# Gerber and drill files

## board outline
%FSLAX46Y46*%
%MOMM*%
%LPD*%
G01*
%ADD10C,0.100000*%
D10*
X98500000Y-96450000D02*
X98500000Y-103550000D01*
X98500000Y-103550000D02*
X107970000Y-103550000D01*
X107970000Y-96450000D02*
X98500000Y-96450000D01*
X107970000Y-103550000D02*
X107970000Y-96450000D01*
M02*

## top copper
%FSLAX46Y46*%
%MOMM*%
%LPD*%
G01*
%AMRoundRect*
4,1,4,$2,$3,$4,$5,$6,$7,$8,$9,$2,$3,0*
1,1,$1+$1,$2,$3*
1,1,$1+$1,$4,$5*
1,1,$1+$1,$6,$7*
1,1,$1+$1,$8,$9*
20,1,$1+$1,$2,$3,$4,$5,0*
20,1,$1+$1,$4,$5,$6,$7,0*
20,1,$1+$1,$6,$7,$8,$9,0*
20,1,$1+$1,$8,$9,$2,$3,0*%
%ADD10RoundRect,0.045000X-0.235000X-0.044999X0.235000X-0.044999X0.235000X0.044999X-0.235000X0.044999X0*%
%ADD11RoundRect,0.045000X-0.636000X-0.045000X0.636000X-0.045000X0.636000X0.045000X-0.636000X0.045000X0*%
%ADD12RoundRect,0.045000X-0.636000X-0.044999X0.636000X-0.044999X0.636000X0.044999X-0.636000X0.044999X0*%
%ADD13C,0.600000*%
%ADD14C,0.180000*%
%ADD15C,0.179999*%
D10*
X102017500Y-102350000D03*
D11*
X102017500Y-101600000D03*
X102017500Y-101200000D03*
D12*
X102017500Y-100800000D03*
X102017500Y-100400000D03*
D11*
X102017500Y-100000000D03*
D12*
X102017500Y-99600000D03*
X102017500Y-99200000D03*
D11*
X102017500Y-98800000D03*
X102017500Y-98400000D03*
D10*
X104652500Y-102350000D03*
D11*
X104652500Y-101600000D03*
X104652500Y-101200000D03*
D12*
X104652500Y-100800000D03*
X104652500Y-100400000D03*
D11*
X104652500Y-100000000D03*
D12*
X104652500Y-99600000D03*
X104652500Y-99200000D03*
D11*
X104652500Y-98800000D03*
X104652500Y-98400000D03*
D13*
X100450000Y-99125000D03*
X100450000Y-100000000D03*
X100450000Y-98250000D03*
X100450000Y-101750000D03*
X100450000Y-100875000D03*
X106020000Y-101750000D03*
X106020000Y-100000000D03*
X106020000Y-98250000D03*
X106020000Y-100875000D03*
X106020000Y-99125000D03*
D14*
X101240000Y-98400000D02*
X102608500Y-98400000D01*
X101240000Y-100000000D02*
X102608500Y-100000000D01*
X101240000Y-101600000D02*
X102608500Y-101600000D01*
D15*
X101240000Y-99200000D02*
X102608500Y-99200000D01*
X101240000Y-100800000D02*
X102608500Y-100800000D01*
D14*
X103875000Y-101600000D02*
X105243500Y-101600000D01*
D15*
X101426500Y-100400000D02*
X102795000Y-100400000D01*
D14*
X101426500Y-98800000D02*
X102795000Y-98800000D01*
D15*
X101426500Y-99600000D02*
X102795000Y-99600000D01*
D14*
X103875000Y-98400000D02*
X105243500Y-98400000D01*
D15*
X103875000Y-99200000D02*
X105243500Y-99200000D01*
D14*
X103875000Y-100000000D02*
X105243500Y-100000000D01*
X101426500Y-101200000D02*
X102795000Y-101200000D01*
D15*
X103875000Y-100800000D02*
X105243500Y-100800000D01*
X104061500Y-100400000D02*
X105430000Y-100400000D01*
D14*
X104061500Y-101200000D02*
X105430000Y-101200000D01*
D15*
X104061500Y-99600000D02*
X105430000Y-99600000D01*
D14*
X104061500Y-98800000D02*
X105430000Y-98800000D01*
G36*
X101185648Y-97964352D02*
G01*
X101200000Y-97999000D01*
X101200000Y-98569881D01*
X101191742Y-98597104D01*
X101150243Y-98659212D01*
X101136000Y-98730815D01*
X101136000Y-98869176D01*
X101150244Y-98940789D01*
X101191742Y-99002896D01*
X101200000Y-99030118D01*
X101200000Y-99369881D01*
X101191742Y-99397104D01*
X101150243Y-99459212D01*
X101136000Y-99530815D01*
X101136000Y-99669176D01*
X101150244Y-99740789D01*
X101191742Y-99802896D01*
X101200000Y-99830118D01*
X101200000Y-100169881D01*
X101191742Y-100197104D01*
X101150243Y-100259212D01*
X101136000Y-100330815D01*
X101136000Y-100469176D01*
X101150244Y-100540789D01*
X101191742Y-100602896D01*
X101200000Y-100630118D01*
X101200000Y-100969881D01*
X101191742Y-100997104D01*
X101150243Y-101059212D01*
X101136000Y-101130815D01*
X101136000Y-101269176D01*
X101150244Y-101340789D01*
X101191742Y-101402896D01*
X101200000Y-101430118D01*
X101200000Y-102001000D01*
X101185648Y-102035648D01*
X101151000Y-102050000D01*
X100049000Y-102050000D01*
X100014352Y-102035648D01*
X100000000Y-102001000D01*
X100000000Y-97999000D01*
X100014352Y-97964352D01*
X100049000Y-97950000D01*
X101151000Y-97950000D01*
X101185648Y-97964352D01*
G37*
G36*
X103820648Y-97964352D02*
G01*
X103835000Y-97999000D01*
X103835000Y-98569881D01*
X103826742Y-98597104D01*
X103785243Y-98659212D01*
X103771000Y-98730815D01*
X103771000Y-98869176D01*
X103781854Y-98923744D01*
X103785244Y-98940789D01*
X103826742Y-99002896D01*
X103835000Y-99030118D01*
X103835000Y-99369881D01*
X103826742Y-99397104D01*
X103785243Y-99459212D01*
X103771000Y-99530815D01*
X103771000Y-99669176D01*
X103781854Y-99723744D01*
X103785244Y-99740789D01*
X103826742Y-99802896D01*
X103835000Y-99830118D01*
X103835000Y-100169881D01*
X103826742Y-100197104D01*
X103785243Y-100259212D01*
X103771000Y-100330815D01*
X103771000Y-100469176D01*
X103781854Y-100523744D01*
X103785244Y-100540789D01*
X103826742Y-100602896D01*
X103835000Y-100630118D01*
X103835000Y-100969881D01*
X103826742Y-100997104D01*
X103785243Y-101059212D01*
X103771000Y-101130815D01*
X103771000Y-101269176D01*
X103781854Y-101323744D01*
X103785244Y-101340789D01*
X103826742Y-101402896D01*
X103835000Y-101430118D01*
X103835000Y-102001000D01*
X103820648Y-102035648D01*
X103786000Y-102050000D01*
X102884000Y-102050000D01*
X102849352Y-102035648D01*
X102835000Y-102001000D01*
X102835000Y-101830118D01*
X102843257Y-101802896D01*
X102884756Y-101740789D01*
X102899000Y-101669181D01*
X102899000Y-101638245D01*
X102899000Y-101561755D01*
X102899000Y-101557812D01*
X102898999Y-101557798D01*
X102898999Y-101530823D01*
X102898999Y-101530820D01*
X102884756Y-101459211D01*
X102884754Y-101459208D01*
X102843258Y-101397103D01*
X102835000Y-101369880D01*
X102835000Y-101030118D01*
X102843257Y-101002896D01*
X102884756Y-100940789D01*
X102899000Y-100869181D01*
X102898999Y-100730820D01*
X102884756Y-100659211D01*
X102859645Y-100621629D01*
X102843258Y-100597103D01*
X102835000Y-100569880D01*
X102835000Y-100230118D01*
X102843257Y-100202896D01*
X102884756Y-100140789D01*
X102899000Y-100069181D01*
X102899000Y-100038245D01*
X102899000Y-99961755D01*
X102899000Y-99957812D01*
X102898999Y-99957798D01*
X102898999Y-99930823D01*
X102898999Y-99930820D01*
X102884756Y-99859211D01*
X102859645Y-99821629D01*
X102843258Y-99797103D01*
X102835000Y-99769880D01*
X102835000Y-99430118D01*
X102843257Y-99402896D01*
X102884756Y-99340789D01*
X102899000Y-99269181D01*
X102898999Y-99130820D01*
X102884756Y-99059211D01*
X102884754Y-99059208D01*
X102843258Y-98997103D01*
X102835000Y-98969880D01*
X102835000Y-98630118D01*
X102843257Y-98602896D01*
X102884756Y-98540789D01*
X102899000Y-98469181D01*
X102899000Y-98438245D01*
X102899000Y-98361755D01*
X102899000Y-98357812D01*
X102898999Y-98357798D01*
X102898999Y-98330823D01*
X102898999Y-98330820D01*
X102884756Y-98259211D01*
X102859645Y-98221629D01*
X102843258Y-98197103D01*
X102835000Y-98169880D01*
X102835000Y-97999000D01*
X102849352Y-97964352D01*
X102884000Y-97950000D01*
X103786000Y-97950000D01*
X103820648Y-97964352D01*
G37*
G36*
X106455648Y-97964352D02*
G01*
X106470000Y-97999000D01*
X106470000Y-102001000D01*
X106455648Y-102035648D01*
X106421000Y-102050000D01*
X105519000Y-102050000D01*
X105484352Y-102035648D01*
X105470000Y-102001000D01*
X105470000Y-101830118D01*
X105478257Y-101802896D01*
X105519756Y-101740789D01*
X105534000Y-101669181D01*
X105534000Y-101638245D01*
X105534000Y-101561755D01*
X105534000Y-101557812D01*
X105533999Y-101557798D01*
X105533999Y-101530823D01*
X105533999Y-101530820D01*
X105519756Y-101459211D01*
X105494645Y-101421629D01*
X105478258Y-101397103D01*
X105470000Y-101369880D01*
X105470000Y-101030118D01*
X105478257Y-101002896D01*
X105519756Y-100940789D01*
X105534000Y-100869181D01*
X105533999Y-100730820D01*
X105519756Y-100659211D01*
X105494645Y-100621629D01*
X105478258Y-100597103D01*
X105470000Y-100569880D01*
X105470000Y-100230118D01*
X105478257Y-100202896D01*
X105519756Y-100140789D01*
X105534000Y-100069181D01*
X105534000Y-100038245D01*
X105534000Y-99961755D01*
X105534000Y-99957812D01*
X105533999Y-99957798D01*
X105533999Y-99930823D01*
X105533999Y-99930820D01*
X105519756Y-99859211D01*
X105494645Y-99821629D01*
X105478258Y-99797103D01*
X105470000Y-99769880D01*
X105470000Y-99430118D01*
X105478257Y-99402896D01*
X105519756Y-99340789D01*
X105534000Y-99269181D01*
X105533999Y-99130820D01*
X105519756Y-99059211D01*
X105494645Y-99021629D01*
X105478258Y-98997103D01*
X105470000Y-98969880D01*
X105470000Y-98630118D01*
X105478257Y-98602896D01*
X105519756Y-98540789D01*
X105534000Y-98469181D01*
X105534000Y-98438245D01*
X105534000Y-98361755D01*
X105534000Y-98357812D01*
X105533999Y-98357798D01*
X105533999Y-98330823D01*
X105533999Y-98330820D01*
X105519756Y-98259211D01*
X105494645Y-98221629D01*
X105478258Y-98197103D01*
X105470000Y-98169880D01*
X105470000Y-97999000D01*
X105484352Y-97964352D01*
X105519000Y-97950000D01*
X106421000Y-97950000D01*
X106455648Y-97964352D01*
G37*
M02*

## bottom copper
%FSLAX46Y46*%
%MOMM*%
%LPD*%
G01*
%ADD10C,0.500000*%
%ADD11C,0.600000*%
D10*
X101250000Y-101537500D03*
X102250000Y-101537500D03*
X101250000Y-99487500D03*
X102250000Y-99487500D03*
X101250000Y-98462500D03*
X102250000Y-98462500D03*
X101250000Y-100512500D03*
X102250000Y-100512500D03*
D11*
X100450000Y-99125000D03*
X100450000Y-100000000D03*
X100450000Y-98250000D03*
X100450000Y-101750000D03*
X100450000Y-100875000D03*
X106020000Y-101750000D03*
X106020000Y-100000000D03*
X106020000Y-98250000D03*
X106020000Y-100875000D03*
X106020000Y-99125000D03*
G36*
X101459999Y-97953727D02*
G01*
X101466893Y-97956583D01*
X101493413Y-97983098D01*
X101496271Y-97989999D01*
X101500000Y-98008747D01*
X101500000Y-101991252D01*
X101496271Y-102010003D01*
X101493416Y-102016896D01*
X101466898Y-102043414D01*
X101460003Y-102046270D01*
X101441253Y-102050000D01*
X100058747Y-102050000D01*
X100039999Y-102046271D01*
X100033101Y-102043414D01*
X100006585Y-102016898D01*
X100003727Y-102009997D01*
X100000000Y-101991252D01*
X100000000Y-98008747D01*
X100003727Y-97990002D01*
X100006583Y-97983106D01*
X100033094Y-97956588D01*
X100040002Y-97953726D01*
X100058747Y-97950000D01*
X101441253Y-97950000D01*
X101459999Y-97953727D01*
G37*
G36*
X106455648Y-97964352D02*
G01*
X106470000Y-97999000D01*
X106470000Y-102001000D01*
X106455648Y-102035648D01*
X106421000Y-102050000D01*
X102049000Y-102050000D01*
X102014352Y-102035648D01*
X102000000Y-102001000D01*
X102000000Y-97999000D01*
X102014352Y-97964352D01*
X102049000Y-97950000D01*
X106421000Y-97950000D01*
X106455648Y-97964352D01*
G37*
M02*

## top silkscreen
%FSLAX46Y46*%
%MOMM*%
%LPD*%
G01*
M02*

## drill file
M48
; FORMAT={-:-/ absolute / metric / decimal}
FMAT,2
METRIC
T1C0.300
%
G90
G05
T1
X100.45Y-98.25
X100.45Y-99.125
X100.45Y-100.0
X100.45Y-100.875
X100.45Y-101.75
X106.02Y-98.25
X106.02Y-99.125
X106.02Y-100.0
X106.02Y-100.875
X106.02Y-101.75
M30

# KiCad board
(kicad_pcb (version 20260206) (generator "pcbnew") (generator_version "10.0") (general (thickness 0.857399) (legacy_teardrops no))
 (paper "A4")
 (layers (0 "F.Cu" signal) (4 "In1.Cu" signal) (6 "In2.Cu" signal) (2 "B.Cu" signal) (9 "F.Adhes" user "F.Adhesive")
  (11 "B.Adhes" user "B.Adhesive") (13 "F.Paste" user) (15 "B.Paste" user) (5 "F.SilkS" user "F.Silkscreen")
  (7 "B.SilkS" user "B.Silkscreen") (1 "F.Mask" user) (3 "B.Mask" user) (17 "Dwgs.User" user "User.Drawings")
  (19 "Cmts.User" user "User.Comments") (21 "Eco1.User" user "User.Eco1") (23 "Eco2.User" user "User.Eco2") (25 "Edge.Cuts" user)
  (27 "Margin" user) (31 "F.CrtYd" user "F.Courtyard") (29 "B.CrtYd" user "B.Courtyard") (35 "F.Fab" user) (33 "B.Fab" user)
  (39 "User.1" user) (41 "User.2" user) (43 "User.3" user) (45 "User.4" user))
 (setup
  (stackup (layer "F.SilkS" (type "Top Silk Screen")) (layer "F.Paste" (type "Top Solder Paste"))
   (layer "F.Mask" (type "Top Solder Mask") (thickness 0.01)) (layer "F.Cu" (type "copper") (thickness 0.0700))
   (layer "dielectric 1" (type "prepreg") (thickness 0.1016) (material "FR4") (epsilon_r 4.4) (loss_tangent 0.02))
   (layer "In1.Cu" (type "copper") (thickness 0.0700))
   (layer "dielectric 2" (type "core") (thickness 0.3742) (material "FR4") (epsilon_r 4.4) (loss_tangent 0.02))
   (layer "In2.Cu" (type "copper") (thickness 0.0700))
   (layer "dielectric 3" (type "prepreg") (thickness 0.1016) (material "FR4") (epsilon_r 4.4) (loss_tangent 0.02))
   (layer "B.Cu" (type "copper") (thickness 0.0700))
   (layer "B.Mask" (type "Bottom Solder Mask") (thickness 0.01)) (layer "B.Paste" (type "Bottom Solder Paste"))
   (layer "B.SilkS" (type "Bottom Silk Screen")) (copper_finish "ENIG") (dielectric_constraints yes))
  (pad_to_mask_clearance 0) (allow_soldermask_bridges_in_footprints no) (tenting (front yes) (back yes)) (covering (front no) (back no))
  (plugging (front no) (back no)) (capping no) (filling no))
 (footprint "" (layer "F.Cu") (at 0 0)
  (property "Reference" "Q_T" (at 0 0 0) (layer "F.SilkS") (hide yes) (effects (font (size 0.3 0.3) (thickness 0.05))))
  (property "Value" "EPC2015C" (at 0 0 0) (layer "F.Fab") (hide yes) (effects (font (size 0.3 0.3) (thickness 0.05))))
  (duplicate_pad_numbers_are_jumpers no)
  (pad "1" smd roundrect (at 102.0175 102.35) (size 0.56 0.179999) (layers "F.Cu" "F.Mask" "F.Paste") (roundrect_rratio 0.25) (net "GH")
   (thermal_bridge_angle 45))
  (pad "3" smd roundrect (at 102.0175 101.6) (size 1.362 0.18) (layers "F.Cu" "F.Mask" "F.Paste") (roundrect_rratio 0.25) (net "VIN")
   (thermal_bridge_angle 45))
  (pad "4" smd roundrect (at 102.0175 101.2) (size 1.362 0.18) (layers "F.Cu" "F.Mask" "F.Paste") (roundrect_rratio 0.25) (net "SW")
   (thermal_bridge_angle 45))
  (pad "5" smd roundrect (at 102.0175 100.8) (size 1.362 0.179999) (layers "F.Cu" "F.Mask" "F.Paste") (roundrect_rratio 0.25) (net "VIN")
   (thermal_bridge_angle 45))
  (pad "6" smd roundrect (at 102.0175 100.4) (size 1.362 0.179999) (layers "F.Cu" "F.Mask" "F.Paste") (roundrect_rratio 0.25) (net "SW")
   (thermal_bridge_angle 45))
  (pad "7" smd roundrect (at 102.0175 100) (size 1.362 0.18) (layers "F.Cu" "F.Mask" "F.Paste") (roundrect_rratio 0.25) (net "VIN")
   (thermal_bridge_angle 45))
  (pad "8" smd roundrect (at 102.0175 99.6) (size 1.362 0.179999) (layers "F.Cu" "F.Mask" "F.Paste") (roundrect_rratio 0.25) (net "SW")
   (thermal_bridge_angle 45))
  (pad "9" smd roundrect (at 102.0175 99.2) (size 1.362 0.179999) (layers "F.Cu" "F.Mask" "F.Paste") (roundrect_rratio 0.25) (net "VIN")
   (thermal_bridge_angle 45))
  (pad "10" smd roundrect (at 102.0175 98.8) (size 1.362 0.18) (layers "F.Cu" "F.Mask" "F.Paste") (roundrect_rratio 0.25) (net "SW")
   (thermal_bridge_angle 45))
  (pad "11" smd roundrect (at 102.0175 98.4) (size 1.362 0.18) (layers "F.Cu" "F.Mask" "F.Paste") (roundrect_rratio 0.25) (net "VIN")
   (thermal_bridge_angle 45)))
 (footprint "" (layer "F.Cu") (at 0 0)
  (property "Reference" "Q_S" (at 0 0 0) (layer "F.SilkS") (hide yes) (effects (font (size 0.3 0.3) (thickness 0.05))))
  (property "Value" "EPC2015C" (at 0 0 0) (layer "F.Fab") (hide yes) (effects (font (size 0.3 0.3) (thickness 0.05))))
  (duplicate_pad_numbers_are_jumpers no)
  (pad "1" smd roundrect (at 104.6525 102.35) (size 0.56 0.179999) (layers "F.Cu" "F.Mask" "F.Paste") (roundrect_rratio 0.25) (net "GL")
   (thermal_bridge_angle 45))
  (pad "3" smd roundrect (at 104.6525 101.6) (size 1.362 0.18) (layers "F.Cu" "F.Mask" "F.Paste") (roundrect_rratio 0.25) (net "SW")
   (thermal_bridge_angle 45))
  (pad "4" smd roundrect (at 104.6525 101.2) (size 1.362 0.18) (layers "F.Cu" "F.Mask" "F.Paste") (roundrect_rratio 0.25) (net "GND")
   (thermal_bridge_angle 45))
  (pad "5" smd roundrect (at 104.6525 100.8) (size 1.362 0.179999) (layers "F.Cu" "F.Mask" "F.Paste") (roundrect_rratio 0.25) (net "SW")
   (thermal_bridge_angle 45))
  (pad "6" smd roundrect (at 104.6525 100.4) (size 1.362 0.179999) (layers "F.Cu" "F.Mask" "F.Paste") (roundrect_rratio 0.25) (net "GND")
   (thermal_bridge_angle 45))
  (pad "7" smd roundrect (at 104.6525 100) (size 1.362 0.18) (layers "F.Cu" "F.Mask" "F.Paste") (roundrect_rratio 0.25) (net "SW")
   (thermal_bridge_angle 45))
  (pad "8" smd roundrect (at 104.6525 99.6) (size 1.362 0.179999) (layers "F.Cu" "F.Mask" "F.Paste") (roundrect_rratio 0.25) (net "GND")
   (thermal_bridge_angle 45))
  (pad "9" smd roundrect (at 104.6525 99.2) (size 1.362 0.179999) (layers "F.Cu" "F.Mask" "F.Paste") (roundrect_rratio 0.25) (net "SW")
   (thermal_bridge_angle 45))
  (pad "10" smd roundrect (at 104.6525 98.8) (size 1.362 0.18) (layers "F.Cu" "F.Mask" "F.Paste") (roundrect_rratio 0.25) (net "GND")
   (thermal_bridge_angle 45))
  (pad "11" smd roundrect (at 104.6525 98.4) (size 1.362 0.18) (layers "F.Cu" "F.Mask" "F.Paste") (roundrect_rratio 0.25) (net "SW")
   (thermal_bridge_angle 45)))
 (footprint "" (layer "B.Cu") (at 101.75 101.5375)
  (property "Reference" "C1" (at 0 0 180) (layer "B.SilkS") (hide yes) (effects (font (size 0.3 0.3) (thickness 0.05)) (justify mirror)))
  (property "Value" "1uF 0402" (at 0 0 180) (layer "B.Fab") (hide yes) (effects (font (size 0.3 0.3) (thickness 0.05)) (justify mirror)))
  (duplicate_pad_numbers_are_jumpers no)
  (pad "1" smd circle (at -0.5 0) (size 0.5 0.5) (layers "B.Cu" "B.Mask" "B.Paste") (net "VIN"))
  (pad "2" smd circle (at 0.5 0) (size 0.5 0.5) (layers "B.Cu" "B.Mask" "B.Paste") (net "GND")))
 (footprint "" (layer "B.Cu") (at 101.75 99.4875)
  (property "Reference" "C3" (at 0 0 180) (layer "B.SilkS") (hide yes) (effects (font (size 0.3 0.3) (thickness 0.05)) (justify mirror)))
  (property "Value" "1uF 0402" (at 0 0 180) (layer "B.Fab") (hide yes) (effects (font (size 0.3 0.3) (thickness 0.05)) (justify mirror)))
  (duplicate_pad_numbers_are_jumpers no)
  (pad "1" smd circle (at -0.5 0) (size 0.5 0.5) (layers "B.Cu" "B.Mask" "B.Paste") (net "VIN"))
  (pad "2" smd circle (at 0.5 0) (size 0.5 0.5) (layers "B.Cu" "B.Mask" "B.Paste") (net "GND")))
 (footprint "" (layer "B.Cu") (at 101.75 98.4625)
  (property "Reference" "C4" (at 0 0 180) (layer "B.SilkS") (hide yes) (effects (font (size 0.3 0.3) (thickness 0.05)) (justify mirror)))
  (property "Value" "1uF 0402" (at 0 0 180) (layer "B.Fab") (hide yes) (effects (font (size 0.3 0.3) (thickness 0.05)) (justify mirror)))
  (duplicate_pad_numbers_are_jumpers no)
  (pad "1" smd circle (at -0.5 0) (size 0.5 0.5) (layers "B.Cu" "B.Mask" "B.Paste") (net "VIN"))
  (pad "2" smd circle (at 0.5 0) (size 0.5 0.5) (layers "B.Cu" "B.Mask" "B.Paste") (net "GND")))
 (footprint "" (layer "B.Cu") (at 101.75 100.5125)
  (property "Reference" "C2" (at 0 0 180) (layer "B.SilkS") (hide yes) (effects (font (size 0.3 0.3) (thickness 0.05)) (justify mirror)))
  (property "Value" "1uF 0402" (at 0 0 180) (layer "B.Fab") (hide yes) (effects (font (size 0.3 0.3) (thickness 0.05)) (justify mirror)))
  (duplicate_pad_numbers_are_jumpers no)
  (pad "1" smd circle (at -0.5 0) (size 0.5 0.5) (layers "B.Cu" "B.Mask" "B.Paste") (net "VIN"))
  (pad "2" smd circle (at 0.5 0) (size 0.5 0.5) (layers "B.Cu" "B.Mask" "B.Paste") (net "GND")))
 (gr_line (start 98.5 96.45) (end 98.5 103.55) (stroke (width 0.1) (type default)) (layer "Edge.Cuts"))
 (gr_line (start 98.5 103.55) (end 107.97 103.55) (stroke (width 0.1) (type default)) (layer "Edge.Cuts"))
 (gr_line (start 107.97 96.45) (end 98.5 96.45) (stroke (width 0.1) (type default)) (layer "Edge.Cuts"))
 (gr_line (start 107.97 103.55) (end 107.97 96.45) (stroke (width 0.1) (type default)) (layer "Edge.Cuts"))
 (segment (start 101.24 98.4) (end 102.6085 98.4) (width 0.18) (layer "F.Cu") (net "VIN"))
 (segment (start 101.24 100) (end 102.6085 100) (width 0.18) (layer "F.Cu") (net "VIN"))
 (segment (start 101.24 101.6) (end 102.6085 101.6) (width 0.18) (layer "F.Cu") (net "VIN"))
 (segment (start 101.24 99.2) (end 102.6085 99.2) (width 0.179999) (layer "F.Cu") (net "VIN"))
 (segment (start 101.24 100.8) (end 102.6085 100.8) (width 0.179999) (layer "F.Cu") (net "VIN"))
 (via (at 100.45 99.125) (size 0.6) (drill 0.3) (layers "F.Cu" "B.Cu") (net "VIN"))
 (via (at 100.45 100) (size 0.6) (drill 0.3) (layers "F.Cu" "B.Cu") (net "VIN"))
 (via (at 100.45 98.25) (size 0.6) (drill 0.3) (layers "F.Cu" "B.Cu") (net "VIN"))
 (via (at 100.45 101.75) (size 0.6) (drill 0.3) (layers "F.Cu" "B.Cu") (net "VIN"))
 (via (at 100.45 100.875) (size 0.6) (drill 0.3) (layers "F.Cu" "B.Cu") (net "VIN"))
 (segment (start 103.875 101.6) (end 105.2435 101.6) (width 0.18) (layer "F.Cu") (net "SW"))
 (segment (start 101.4265 100.4) (end 102.795 100.4) (width 0.179999) (layer "F.Cu") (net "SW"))
 (segment (start 101.4265 98.8) (end 102.795 98.8) (width 0.18) (layer "F.Cu") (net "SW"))
 (segment (start 101.4265 99.6) (end 102.795 99.6) (width 0.179999) (layer "F.Cu") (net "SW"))
 (segment (start 103.875 98.4) (end 105.2435 98.4) (width 0.18) (layer "F.Cu") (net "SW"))
 (segment (start 103.875 99.2) (end 105.2435 99.2) (width 0.179999) (layer "F.Cu") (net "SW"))
 (segment (start 103.875 100) (end 105.2435 100) (width 0.18) (layer "F.Cu") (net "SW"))
 (segment (start 101.4265 101.2) (end 102.795 101.2) (width 0.18) (layer "F.Cu") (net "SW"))
 (segment (start 103.875 100.8) (end 105.2435 100.8) (width 0.179999) (layer "F.Cu") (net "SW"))
 (segment (start 104.0615 100.4) (end 105.43 100.4) (width 0.179999) (layer "F.Cu") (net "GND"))
 (segment (start 104.0615 101.2) (end 105.43 101.2) (width 0.18) (layer "F.Cu") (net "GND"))
 (segment (start 104.0615 99.6) (end 105.43 99.6) (width 0.179999) (layer "F.Cu") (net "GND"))
 (segment (start 104.0615 98.8) (end 105.43 98.8) (width 0.18) (layer "F.Cu") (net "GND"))
 (via (at 106.02 101.75) (size 0.6) (drill 0.3) (layers "F.Cu" "B.Cu") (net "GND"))
 (via (at 106.02 100) (size 0.6) (drill 0.3) (layers "F.Cu" "B.Cu") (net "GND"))
 (via (at 106.02 98.25) (size 0.6) (drill 0.3) (layers "F.Cu" "B.Cu") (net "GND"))
 (via (at 106.02 100.875) (size 0.6) (drill 0.3) (layers "F.Cu" "B.Cu") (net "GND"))
 (via (at 106.02 99.125) (size 0.6) (drill 0.3) (layers "F.Cu" "B.Cu") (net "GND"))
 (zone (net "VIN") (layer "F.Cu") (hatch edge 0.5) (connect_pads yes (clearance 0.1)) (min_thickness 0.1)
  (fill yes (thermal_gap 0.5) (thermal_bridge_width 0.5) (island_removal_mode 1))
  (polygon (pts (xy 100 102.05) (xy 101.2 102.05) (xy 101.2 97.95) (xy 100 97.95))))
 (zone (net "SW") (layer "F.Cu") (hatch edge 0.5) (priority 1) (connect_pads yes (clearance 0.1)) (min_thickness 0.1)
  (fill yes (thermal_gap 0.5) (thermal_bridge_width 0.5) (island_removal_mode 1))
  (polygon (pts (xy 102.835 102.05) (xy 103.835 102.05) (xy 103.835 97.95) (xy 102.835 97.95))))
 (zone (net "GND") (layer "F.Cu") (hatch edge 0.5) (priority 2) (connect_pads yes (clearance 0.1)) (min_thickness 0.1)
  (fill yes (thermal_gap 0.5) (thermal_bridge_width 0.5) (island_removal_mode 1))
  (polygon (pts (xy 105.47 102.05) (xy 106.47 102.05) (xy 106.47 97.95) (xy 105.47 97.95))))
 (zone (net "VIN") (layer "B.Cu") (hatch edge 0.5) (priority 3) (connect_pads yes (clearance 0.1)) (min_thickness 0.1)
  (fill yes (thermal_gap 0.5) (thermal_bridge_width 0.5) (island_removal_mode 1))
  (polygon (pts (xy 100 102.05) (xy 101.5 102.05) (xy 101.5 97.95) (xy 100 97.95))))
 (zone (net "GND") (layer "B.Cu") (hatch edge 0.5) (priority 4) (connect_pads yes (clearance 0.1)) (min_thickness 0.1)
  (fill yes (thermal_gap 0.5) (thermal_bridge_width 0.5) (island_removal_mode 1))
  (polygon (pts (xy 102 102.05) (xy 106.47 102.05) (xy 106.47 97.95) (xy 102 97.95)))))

